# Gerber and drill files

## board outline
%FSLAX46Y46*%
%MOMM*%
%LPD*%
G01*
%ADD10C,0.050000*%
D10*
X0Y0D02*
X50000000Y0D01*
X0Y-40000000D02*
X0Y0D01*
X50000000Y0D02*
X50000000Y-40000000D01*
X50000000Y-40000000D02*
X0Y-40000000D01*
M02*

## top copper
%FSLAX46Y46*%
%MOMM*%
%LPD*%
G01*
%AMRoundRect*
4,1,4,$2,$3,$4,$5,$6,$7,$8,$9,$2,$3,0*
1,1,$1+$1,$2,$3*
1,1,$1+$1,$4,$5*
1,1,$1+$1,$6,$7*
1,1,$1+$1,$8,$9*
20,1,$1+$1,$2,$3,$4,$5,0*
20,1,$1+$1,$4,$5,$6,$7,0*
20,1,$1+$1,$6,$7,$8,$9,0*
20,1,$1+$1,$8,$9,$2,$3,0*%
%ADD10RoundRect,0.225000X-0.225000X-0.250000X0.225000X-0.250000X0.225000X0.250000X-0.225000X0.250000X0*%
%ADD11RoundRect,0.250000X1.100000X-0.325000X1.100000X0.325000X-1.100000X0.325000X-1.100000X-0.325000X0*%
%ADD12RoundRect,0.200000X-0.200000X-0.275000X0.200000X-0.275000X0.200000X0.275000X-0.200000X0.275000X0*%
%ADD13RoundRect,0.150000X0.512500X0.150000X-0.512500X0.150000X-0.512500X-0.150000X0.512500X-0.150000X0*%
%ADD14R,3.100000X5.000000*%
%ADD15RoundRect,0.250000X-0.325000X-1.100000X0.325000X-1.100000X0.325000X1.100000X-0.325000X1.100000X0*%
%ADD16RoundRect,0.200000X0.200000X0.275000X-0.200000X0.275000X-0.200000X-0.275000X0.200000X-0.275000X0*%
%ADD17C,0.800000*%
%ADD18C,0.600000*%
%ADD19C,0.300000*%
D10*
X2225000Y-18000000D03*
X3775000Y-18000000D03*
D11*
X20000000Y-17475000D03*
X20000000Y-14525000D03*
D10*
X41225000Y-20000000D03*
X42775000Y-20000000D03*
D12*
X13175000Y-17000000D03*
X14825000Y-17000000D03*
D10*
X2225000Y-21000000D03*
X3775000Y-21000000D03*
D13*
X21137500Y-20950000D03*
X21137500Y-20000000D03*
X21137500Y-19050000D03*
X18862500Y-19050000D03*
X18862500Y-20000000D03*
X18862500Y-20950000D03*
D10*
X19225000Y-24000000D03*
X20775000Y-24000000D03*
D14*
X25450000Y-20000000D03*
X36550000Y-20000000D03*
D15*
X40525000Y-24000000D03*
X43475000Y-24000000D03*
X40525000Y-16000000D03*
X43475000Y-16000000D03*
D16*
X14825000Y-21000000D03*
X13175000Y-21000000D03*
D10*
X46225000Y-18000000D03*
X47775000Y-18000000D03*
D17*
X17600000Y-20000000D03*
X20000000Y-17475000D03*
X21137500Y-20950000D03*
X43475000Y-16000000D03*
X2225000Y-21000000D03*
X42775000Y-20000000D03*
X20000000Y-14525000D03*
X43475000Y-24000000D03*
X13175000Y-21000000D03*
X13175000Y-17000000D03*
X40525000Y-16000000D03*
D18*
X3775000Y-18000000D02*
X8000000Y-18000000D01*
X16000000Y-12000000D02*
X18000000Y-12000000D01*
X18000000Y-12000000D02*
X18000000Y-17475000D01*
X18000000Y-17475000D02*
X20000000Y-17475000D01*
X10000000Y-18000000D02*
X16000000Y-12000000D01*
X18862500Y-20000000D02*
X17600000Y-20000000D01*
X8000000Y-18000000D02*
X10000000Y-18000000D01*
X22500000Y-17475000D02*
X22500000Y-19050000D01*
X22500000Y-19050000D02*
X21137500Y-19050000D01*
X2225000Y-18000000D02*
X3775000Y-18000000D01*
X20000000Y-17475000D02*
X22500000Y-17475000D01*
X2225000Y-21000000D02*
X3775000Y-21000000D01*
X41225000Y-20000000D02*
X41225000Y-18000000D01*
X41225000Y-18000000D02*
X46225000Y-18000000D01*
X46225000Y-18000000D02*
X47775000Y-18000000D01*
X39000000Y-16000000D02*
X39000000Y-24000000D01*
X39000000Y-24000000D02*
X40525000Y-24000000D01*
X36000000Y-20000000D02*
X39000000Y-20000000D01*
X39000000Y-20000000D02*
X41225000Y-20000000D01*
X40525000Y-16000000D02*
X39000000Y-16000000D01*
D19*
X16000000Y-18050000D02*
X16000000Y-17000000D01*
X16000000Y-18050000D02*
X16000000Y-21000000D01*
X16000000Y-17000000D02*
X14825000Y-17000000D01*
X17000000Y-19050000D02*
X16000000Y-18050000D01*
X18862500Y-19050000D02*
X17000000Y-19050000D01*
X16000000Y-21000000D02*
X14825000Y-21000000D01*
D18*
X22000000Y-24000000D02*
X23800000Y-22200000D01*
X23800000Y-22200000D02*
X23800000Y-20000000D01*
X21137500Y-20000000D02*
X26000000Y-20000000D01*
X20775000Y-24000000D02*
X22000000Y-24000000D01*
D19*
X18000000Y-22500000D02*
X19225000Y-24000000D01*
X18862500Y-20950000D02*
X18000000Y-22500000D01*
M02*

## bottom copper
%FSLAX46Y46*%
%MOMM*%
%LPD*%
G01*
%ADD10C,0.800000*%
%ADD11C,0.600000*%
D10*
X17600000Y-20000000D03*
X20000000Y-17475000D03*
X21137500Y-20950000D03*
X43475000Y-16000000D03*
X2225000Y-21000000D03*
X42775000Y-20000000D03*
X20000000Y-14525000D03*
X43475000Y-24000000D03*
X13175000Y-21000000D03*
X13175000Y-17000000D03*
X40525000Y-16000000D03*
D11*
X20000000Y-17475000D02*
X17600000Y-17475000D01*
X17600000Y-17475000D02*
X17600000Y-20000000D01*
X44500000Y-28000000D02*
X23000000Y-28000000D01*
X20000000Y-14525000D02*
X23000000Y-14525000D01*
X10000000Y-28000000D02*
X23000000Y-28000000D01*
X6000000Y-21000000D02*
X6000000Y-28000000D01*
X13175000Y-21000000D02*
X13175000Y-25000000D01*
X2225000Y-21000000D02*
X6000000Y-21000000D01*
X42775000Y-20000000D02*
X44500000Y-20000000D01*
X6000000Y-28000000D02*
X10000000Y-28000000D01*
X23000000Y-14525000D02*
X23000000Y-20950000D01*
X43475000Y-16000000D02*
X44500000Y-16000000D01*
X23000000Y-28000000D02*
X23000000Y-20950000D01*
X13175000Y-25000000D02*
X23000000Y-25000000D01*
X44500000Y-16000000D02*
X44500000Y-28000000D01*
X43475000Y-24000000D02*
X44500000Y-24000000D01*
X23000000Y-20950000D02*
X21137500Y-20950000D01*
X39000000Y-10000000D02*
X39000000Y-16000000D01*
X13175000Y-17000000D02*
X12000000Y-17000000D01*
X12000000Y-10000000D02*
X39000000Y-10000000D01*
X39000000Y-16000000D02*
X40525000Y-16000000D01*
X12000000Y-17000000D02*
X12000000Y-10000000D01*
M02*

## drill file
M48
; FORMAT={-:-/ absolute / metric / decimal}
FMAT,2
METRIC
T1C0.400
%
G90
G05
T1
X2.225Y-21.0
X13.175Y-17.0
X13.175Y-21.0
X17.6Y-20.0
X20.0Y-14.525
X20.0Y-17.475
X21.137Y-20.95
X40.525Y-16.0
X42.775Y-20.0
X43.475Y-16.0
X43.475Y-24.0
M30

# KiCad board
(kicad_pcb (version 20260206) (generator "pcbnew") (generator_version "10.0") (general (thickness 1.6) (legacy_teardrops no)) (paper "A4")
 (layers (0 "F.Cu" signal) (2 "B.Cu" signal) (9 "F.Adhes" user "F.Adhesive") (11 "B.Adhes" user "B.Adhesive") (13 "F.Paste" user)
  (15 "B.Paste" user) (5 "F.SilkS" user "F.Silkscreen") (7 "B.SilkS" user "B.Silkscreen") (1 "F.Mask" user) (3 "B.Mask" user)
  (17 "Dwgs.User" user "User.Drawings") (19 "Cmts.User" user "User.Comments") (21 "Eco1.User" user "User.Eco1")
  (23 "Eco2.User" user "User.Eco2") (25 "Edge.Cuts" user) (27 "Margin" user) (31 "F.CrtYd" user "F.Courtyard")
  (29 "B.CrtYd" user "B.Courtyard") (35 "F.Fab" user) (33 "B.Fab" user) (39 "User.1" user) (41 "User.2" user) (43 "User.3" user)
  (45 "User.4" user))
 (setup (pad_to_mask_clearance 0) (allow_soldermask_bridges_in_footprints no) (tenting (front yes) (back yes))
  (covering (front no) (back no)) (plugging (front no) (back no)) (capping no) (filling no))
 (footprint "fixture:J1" (layer "F.Cu") (at 3 18)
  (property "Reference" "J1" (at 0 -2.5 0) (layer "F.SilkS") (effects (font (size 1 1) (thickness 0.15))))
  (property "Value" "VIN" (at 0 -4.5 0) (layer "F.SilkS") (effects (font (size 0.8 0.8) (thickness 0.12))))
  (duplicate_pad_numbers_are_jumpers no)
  (pad "1" smd roundrect (at -0.775 0) (size 0.9 0.95) (layers "F.Cu" "F.Mask" "F.Paste") (roundrect_rratio 0.25) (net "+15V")
   (thermal_bridge_angle 45))
  (pad "2" smd roundrect (at 0.775 0) (size 0.9 0.95) (layers "F.Cu" "F.Mask" "F.Paste") (roundrect_rratio 0.25) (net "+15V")
   (thermal_bridge_angle 45)))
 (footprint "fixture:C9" (layer "F.Cu") (at 20 16 90)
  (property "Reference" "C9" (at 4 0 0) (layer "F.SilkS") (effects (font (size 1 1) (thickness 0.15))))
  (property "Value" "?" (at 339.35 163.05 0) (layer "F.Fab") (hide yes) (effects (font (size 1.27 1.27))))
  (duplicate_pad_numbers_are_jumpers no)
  (pad "1" smd roundrect (at -1.475 0 90) (size 1.15 2.7) (layers "F.Cu" "F.Mask" "F.Paste") (roundrect_rratio 0.217391) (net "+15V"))
  (pad "2" smd roundrect (at 1.475 0 90) (size 1.15 2.7) (layers "F.Cu" "F.Mask" "F.Paste") (roundrect_rratio 0.217391) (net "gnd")))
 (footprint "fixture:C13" (layer "F.Cu") (at 42 20)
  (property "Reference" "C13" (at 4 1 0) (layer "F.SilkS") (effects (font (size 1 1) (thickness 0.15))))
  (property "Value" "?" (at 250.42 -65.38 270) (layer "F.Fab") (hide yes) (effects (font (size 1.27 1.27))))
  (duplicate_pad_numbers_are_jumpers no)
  (pad "1" smd roundrect (at -0.775 0) (size 0.9 0.95) (layers "F.Cu" "F.Mask" "F.Paste") (roundrect_rratio 0.25) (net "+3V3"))
  (pad "2" smd roundrect (at 0.775 0) (size 0.9 0.95) (layers "F.Cu" "F.Mask" "F.Paste") (roundrect_rratio 0.25) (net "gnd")))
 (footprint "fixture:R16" (layer "F.Cu") (at 14 17)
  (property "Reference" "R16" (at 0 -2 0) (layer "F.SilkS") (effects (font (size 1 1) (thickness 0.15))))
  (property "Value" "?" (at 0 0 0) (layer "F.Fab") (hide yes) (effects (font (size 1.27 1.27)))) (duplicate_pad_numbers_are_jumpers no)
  (pad "1" smd roundrect (at -0.825 0) (size 0.8 0.95) (layers "F.Cu" "F.Mask" "F.Paste") (roundrect_rratio 0.25) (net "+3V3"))
  (pad "2" smd roundrect (at 0.825 0) (size 0.8 0.95) (layers "F.Cu" "F.Mask" "F.Paste") (roundrect_rratio 0.25) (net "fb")))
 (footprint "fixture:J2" (layer "F.Cu") (at 3 21)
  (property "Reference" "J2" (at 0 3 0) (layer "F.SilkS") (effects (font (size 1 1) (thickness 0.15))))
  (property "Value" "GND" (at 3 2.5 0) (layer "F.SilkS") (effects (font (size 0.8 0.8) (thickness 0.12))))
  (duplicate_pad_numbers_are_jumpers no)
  (pad "1" smd roundrect (at -0.775 0) (size 0.9 0.95) (layers "F.Cu" "F.Mask" "F.Paste") (roundrect_rratio 0.25) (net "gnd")
   (thermal_bridge_angle 45))
  (pad "2" smd roundrect (at 0.775 0) (size 0.9 0.95) (layers "F.Cu" "F.Mask" "F.Paste") (roundrect_rratio 0.25) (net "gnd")
   (thermal_bridge_angle 45)))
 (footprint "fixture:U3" (layer "F.Cu") (at 20 20 180)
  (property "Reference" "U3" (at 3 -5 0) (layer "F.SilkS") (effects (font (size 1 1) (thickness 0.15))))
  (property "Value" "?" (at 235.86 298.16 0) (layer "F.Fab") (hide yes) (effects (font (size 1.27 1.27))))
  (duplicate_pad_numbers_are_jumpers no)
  (pad "1" smd roundrect (at -1.1375 -0.95 180) (size 1.325 0.6) (layers "F.Cu" "F.Mask" "F.Paste") (roundrect_rratio 0.25) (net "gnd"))
  (pad "2" smd roundrect (at -1.1375 0 180) (size 1.325 0.6) (layers "F.Cu" "F.Mask" "F.Paste") (roundrect_rratio 0.25) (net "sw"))
  (pad "3" smd roundrect (at -1.1375 0.95 180) (size 1.325 0.6) (layers "F.Cu" "F.Mask" "F.Paste") (roundrect_rratio 0.25) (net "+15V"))
  (pad "4" smd roundrect (at 1.1375 0.95 180) (size 1.325 0.6) (layers "F.Cu" "F.Mask" "F.Paste") (roundrect_rratio 0.25) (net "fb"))
  (pad "5" smd roundrect (at 1.1375 0 180) (size 1.325 0.6) (layers "F.Cu" "F.Mask" "F.Paste") (roundrect_rratio 0.25) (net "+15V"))
  (pad "6" smd roundrect (at 1.1375 -0.95 180) (size 1.325 0.6) (layers "F.Cu" "F.Mask" "F.Paste") (roundrect_rratio 0.25) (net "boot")))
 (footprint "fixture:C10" (layer "F.Cu") (at 20 24)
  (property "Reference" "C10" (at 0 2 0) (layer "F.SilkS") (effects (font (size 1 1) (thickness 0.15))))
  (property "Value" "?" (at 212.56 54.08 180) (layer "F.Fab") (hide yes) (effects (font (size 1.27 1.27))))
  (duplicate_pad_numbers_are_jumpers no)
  (pad "1" smd roundrect (at -0.775 0) (size 0.9 0.95) (layers "F.Cu" "F.Mask" "F.Paste") (roundrect_rratio 0.25) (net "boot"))
  (pad "2" smd roundrect (at 0.775 0) (size 0.9 0.95) (layers "F.Cu" "F.Mask" "F.Paste") (roundrect_rratio 0.25) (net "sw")))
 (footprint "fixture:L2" (layer "F.Cu") (at 31 20)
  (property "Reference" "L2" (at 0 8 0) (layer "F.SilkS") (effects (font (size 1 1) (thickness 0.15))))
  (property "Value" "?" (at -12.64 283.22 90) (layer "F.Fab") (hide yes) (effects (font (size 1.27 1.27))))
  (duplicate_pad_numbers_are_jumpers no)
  (pad "1" smd rect (at -5.55 0) (size 3.1 5) (layers "F.Cu" "F.Mask" "F.Paste") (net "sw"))
  (pad "2" smd rect (at 5.55 0) (size 3.1 5) (layers "F.Cu" "F.Mask" "F.Paste") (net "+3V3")))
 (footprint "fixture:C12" (layer "F.Cu") (at 42 24)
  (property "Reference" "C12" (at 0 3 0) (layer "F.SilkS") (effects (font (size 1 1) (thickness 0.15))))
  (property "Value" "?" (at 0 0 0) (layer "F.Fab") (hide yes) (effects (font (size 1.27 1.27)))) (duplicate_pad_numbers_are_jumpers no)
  (pad "1" smd roundrect (at -1.475 0) (size 1.15 2.7) (layers "F.Cu" "F.Mask" "F.Paste") (roundrect_rratio 0.217391) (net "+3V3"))
  (pad "2" smd roundrect (at 1.475 0) (size 1.15 2.7) (layers "F.Cu" "F.Mask" "F.Paste") (roundrect_rratio 0.217391) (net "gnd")))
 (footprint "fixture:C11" (layer "F.Cu") (at 42 16)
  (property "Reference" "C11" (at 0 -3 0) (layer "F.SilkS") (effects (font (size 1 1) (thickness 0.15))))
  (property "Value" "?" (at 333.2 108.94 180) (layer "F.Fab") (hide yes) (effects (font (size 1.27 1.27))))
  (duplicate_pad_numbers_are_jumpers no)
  (pad "1" smd roundrect (at -1.475 0) (size 1.15 2.7) (layers "F.Cu" "F.Mask" "F.Paste") (roundrect_rratio 0.217391) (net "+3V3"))
  (pad "2" smd roundrect (at 1.475 0) (size 1.15 2.7) (layers "F.Cu" "F.Mask" "F.Paste") (roundrect_rratio 0.217391) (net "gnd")))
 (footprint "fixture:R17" (layer "F.Cu") (at 14 21 180)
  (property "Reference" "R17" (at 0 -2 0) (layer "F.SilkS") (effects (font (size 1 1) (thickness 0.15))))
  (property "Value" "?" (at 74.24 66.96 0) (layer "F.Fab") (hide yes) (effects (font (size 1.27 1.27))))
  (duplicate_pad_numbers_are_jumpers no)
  (pad "1" smd roundrect (at -0.825 0 180) (size 0.8 0.95) (layers "F.Cu" "F.Mask" "F.Paste") (roundrect_rratio 0.25) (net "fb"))
  (pad "2" smd roundrect (at 0.825 0 180) (size 0.8 0.95) (layers "F.Cu" "F.Mask" "F.Paste") (roundrect_rratio 0.25) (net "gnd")))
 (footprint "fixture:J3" (layer "F.Cu") (at 47 18)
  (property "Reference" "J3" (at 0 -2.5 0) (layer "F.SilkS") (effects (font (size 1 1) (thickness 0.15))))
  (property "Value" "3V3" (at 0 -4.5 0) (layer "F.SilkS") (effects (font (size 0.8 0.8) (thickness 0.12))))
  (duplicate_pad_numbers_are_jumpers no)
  (pad "1" smd roundrect (at -0.775 0) (size 0.9 0.95) (layers "F.Cu" "F.Mask" "F.Paste") (roundrect_rratio 0.25) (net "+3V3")
   (thermal_bridge_angle 45))
  (pad "2" smd roundrect (at 0.775 0) (size 0.9 0.95) (layers "F.Cu" "F.Mask" "F.Paste") (roundrect_rratio 0.25) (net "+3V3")
   (thermal_bridge_angle 45)))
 (gr_line (start 0 0) (end 50 0) (stroke (width 0.05) (type default)) (layer "Edge.Cuts"))
 (gr_line (start 0 40) (end 0 0) (stroke (width 0.05) (type default)) (layer "Edge.Cuts"))
 (gr_line (start 50 0) (end 50 40) (stroke (width 0.05) (type default)) (layer "Edge.Cuts"))
 (gr_line (start 50 40) (end 0 40) (stroke (width 0.05) (type default)) (layer "Edge.Cuts"))
 (segment (start 3.775 18) (end 8 18) (width 0.6) (layer "F.Cu") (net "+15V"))
 (segment (start 16 12) (end 18 12) (width 0.6) (layer "F.Cu") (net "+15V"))
 (segment (start 18 12) (end 18 17.475) (width 0.6) (layer "F.Cu") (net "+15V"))
 (segment (start 18 17.475) (end 20 17.475) (width 0.6) (layer "F.Cu") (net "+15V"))
 (segment (start 10 18) (end 16 12) (width 0.6) (layer "F.Cu") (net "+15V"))
 (segment (start 18.8625 20) (end 17.6 20) (width 0.6) (layer "F.Cu") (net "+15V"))
 (segment (start 8 18) (end 10 18) (width 0.6) (layer "F.Cu") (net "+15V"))
 (segment (start 22.5 17.475) (end 22.5 19.05) (width 0.6) (layer "F.Cu") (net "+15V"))
 (segment (start 22.5 19.05) (end 21.1375 19.05) (width 0.6) (layer "F.Cu") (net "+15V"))
 (segment (start 2.225 18) (end 3.775 18) (width 0.6) (layer "F.Cu") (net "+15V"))
 (segment (start 20 17.475) (end 22.5 17.475) (width 0.6) (layer "F.Cu") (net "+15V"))
 (via (at 17.6 20) (size 0.8) (drill 0.4) (layers "F.Cu" "B.Cu") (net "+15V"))
 (via (at 20 17.475) (size 0.8) (drill 0.4) (layers "F.Cu" "B.Cu") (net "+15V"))
 (segment (start 20 17.475) (end 17.6 17.475) (width 0.6) (layer "B.Cu") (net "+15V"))
 (segment (start 17.6 17.475) (end 17.6 20) (width 0.6) (layer "B.Cu") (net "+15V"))
 (segment (start 2.225 21) (end 3.775 21) (width 0.6) (layer "F.Cu") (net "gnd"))
 (via (at 21.1375 20.95) (size 0.8) (drill 0.4) (layers "F.Cu" "B.Cu") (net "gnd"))
 (via (at 43.475 16) (size 0.8) (drill 0.4) (layers "F.Cu" "B.Cu") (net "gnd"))
 (via (at 2.225 21) (size 0.8) (drill 0.4) (layers "F.Cu" "B.Cu") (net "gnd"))
 (via (at 42.775 20) (size 0.8) (drill 0.4) (layers "F.Cu" "B.Cu") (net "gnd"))
 (via (at 20 14.525) (size 0.8) (drill 0.4) (layers "F.Cu" "B.Cu") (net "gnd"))
 (via (at 43.475 24) (size 0.8) (drill 0.4) (layers "F.Cu" "B.Cu") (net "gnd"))
 (via (at 13.175 21) (size 0.8) (drill 0.4) (layers "F.Cu" "B.Cu") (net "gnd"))
 (segment (start 44.5 28) (end 23 28) (width 0.6) (layer "B.Cu") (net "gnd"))
 (segment (start 20 14.525) (end 23 14.525) (width 0.6) (layer "B.Cu") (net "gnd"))
 (segment (start 10 28) (end 23 28) (width 0.6) (layer "B.Cu") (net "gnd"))
 (segment (start 6 21) (end 6 28) (width 0.6) (layer "B.Cu") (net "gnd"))
 (segment (start 13.175 21) (end 13.175 25) (width 0.6) (layer "B.Cu") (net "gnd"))
 (segment (start 2.225 21) (end 6 21) (width 0.6) (layer "B.Cu") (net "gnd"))
 (segment (start 42.775 20) (end 44.5 20) (width 0.6) (layer "B.Cu") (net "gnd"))
 (segment (start 6 28) (end 10 28) (width 0.6) (layer "B.Cu") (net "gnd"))
 (segment (start 23 14.525) (end 23 20.95) (width 0.6) (layer "B.Cu") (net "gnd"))
 (segment (start 43.475 16) (end 44.5 16) (width 0.6) (layer "B.Cu") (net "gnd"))
 (segment (start 23 28) (end 23 20.95) (width 0.6) (layer "B.Cu") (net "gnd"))
 (segment (start 13.175 25) (end 23 25) (width 0.6) (layer "B.Cu") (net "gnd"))
 (segment (start 44.5 16) (end 44.5 28) (width 0.6) (layer "B.Cu") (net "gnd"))
 (segment (start 43.475 24) (end 44.5 24) (width 0.6) (layer "B.Cu") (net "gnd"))
 (segment (start 23 20.95) (end 21.1375 20.95) (width 0.6) (layer "B.Cu") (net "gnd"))
 (segment (start 41.225 20) (end 41.225 18) (width 0.6) (layer "F.Cu") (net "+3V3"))
 (segment (start 41.225 18) (end 46.225 18) (width 0.6) (layer "F.Cu") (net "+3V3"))
 (segment (start 46.225 18) (end 47.775 18) (width 0.6) (layer "F.Cu") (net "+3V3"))
 (segment (start 39 16) (end 39 24) (width 0.6) (layer "F.Cu") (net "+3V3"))
 (segment (start 39 24) (end 40.525 24) (width 0.6) (layer "F.Cu") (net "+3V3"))
 (segment (start 36 20) (end 39 20) (width 0.6) (layer "F.Cu") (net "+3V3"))
 (segment (start 39 20) (end 41.225 20) (width 0.6) (layer "F.Cu") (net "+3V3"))
 (segment (start 40.525 16) (end 39 16) (width 0.6) (layer "F.Cu") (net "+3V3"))
 (via (at 13.175 17) (size 0.8) (drill 0.4) (layers "F.Cu" "B.Cu") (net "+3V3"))
 (via (at 40.525 16) (size 0.8) (drill 0.4) (layers "F.Cu" "B.Cu") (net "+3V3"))
 (segment (start 39 10) (end 39 16) (width 0.6) (layer "B.Cu") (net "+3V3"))
 (segment (start 13.175 17) (end 12 17) (width 0.6) (layer "B.Cu") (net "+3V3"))
 (segment (start 12 10) (end 39 10) (width 0.6) (layer "B.Cu") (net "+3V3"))
 (segment (start 39 16) (end 40.525 16) (width 0.6) (layer "B.Cu") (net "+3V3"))
 (segment (start 12 17) (end 12 10) (width 0.6) (layer "B.Cu") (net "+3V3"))
 (segment (start 16 18.05) (end 16 17) (width 0.3) (layer "F.Cu") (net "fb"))
 (segment (start 16 18.05) (end 16 21) (width 0.3) (layer "F.Cu") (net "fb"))
 (segment (start 16 17) (end 14.825 17) (width 0.3) (layer "F.Cu") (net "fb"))
 (segment (start 17 19.05) (end 16 18.05) (width 0.3) (layer "F.Cu") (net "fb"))
 (segment (start 18.8625 19.05) (end 17 19.05) (width 0.3) (layer "F.Cu") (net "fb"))
 (segment (start 16 21) (end 14.825 21) (width 0.3) (layer "F.Cu") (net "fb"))
 (segment (start 22 24) (end 23.8 22.2) (width 0.6) (layer "F.Cu") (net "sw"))
 (segment (start 23.8 22.2) (end 23.8 20) (width 0.6) (layer "F.Cu") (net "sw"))
 (segment (start 21.1375 20) (end 26 20) (width 0.6) (layer "F.Cu") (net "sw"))
 (segment (start 20.775 24) (end 22 24) (width 0.6) (layer "F.Cu") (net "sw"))
 (segment (start 18 22.5) (end 19.225 24) (width 0.3) (layer "F.Cu") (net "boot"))
 (segment (start 18.8625 20.95) (end 18 22.5) (width 0.3) (layer "F.Cu") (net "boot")))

